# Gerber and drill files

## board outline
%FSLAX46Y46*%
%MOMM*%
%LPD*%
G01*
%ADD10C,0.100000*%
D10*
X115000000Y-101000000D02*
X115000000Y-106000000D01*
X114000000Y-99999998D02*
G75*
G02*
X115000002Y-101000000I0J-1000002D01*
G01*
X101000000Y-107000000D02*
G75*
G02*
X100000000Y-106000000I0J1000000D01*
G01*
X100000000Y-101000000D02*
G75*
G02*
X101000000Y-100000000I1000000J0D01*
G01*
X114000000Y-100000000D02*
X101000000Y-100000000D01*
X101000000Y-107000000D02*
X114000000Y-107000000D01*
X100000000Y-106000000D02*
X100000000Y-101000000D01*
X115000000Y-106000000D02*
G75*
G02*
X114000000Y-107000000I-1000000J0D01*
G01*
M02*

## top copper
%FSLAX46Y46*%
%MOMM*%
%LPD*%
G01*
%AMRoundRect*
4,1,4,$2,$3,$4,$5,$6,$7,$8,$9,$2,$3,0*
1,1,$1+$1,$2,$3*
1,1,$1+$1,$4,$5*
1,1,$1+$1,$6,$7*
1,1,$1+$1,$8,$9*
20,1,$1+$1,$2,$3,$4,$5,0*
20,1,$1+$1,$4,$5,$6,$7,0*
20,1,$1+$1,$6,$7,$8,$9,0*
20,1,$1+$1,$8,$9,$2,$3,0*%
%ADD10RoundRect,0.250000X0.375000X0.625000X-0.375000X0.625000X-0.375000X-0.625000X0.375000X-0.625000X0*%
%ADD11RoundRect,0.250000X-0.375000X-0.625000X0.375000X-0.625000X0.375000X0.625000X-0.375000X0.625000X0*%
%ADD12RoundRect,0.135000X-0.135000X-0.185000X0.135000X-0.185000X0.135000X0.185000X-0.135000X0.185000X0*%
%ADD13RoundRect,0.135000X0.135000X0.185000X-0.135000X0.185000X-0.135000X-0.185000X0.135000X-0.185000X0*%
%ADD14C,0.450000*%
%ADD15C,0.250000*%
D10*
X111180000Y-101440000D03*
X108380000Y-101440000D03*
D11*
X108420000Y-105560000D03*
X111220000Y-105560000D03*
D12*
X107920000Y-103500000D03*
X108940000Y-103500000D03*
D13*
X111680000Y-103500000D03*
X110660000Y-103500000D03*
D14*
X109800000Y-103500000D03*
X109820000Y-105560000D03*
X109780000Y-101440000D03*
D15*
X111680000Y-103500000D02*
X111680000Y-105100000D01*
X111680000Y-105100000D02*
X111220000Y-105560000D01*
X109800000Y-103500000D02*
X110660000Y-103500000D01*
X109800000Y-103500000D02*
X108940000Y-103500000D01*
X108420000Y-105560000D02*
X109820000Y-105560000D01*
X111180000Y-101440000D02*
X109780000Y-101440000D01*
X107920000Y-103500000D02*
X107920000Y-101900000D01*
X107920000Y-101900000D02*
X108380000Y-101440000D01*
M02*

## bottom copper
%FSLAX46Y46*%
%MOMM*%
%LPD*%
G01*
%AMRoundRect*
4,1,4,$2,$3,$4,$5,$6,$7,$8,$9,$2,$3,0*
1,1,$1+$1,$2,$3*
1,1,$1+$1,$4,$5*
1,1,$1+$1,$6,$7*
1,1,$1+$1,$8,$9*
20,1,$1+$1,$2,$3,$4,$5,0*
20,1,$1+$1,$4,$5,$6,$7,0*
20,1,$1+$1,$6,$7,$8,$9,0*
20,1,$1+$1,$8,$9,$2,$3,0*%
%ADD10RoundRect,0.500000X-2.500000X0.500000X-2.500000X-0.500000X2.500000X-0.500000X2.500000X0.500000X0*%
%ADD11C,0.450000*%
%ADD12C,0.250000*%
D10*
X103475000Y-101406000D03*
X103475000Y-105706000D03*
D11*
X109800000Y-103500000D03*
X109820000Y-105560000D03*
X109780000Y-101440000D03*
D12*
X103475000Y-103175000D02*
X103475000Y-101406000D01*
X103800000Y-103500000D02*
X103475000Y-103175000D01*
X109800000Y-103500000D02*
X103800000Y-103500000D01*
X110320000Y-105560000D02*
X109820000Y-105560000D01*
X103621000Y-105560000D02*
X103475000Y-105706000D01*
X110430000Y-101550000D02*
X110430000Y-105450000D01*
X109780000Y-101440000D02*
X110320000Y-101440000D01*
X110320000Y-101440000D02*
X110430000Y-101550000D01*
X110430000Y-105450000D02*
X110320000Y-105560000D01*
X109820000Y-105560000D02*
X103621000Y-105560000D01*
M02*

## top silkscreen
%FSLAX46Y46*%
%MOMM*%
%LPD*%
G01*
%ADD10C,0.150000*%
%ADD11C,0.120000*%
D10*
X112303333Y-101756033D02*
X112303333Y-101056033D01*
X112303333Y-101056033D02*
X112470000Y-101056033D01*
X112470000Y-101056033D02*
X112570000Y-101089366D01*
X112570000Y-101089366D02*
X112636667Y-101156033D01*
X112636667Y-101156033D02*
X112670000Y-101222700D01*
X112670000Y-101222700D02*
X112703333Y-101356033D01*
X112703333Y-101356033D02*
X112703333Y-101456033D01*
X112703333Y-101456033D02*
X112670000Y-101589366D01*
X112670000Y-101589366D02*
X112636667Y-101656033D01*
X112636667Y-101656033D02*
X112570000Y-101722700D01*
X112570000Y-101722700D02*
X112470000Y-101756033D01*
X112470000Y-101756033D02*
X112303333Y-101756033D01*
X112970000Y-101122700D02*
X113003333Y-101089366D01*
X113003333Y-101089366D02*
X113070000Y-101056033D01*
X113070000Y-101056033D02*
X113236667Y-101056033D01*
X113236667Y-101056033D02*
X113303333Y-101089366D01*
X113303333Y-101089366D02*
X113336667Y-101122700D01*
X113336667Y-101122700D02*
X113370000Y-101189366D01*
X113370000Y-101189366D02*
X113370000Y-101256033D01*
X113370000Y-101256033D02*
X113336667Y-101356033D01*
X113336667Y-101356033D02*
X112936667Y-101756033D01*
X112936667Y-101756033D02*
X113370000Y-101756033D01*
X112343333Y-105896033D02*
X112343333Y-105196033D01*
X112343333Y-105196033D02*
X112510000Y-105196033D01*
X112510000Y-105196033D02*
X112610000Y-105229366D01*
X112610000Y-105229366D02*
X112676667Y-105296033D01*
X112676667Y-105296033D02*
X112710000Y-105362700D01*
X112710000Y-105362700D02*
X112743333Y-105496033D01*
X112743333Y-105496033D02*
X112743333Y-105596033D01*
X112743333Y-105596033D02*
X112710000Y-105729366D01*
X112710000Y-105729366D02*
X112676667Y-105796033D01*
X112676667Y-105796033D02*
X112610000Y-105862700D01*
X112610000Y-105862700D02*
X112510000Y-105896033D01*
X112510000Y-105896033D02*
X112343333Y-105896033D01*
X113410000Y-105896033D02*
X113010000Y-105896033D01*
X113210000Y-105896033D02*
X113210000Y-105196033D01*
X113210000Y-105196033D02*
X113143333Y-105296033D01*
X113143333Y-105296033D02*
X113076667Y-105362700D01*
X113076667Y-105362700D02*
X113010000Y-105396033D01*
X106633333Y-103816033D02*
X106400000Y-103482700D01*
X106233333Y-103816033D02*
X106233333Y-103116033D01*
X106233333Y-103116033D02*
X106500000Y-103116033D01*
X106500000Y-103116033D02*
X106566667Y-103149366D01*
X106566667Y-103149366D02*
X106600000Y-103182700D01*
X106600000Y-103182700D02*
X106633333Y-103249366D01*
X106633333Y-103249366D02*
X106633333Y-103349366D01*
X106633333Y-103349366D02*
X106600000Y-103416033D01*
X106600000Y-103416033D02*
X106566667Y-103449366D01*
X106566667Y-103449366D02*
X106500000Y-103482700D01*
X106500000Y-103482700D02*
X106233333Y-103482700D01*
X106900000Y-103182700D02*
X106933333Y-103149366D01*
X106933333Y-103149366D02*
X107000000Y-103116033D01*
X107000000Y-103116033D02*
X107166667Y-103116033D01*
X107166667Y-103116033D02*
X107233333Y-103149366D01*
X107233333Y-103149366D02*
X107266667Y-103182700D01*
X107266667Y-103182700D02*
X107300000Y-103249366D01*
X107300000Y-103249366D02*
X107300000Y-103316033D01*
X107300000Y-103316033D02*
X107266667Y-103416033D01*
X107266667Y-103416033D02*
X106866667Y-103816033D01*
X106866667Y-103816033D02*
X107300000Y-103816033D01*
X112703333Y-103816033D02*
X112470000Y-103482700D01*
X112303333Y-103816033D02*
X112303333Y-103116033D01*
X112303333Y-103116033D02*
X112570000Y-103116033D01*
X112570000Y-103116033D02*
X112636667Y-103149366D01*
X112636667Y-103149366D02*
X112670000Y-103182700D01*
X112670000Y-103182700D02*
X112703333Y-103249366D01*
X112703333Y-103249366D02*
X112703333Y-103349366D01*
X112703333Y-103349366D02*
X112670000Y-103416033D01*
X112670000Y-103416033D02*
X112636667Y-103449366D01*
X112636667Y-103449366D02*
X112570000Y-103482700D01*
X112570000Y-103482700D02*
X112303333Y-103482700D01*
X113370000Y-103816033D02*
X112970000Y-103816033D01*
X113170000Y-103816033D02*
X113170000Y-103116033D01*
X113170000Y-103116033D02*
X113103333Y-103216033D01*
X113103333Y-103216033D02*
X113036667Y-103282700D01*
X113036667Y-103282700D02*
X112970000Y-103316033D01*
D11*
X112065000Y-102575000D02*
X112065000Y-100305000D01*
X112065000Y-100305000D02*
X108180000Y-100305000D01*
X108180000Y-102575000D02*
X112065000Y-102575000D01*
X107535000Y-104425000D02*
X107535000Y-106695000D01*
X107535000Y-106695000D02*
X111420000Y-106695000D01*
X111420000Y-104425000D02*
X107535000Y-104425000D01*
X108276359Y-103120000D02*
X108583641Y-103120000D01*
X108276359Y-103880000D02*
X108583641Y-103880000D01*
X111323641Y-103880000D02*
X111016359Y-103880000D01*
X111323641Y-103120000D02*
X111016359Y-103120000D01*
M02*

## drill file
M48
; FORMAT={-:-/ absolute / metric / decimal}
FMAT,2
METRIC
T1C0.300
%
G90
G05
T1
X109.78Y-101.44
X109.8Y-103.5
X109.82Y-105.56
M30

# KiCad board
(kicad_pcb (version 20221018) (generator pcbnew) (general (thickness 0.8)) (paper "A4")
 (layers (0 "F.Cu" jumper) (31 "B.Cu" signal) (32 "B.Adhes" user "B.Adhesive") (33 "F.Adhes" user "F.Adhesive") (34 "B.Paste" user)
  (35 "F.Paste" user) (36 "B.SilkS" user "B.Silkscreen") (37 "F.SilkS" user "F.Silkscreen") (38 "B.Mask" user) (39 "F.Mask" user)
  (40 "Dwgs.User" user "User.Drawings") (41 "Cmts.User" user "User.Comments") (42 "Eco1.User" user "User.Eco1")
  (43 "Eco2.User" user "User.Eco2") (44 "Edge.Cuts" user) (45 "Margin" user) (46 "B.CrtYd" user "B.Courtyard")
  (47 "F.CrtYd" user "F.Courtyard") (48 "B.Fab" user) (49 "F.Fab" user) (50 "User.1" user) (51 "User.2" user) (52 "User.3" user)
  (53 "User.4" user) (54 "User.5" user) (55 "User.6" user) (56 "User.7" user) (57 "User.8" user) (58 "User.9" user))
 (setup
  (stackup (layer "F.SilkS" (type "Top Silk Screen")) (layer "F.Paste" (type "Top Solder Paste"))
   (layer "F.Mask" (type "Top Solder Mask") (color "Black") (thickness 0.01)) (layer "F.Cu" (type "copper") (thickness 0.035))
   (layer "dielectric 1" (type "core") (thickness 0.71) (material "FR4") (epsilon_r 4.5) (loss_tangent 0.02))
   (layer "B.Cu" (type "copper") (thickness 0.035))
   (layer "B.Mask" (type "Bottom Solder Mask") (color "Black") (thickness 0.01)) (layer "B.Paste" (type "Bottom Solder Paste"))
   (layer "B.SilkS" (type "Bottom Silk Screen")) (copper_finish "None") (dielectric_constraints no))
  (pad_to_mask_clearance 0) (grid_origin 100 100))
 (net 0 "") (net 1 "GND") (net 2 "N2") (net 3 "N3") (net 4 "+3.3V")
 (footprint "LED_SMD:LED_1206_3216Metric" (layer "F.Cu") (at 109.78 101.44 180)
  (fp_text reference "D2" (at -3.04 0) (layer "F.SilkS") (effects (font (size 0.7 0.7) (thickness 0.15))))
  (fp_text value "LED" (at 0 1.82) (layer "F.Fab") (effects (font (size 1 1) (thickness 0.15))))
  (fp_line (start -2.285 -1.135) (end -2.285 1.135) (stroke (width 0.12) (type solid)) (layer "F.SilkS"))
  (fp_line (start -2.285 1.135) (end 1.6 1.135) (stroke (width 0.12) (type solid)) (layer "F.SilkS"))
  (fp_line (start 1.6 -1.135) (end -2.285 -1.135) (stroke (width 0.12) (type solid)) (layer "F.SilkS"))
  (pad "1" smd roundrect (at -1.4 0 180) (size 1.25 1.75) (layers "F.Cu" "F.Paste" "F.Mask") (roundrect_rratio 0.2) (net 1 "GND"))
  (pad "2" smd roundrect (at 1.4 0 180) (size 1.25 1.75) (layers "F.Cu" "F.Paste" "F.Mask") (roundrect_rratio 0.2) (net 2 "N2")))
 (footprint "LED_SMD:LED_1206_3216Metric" (layer "F.Cu") (at 109.82 105.56)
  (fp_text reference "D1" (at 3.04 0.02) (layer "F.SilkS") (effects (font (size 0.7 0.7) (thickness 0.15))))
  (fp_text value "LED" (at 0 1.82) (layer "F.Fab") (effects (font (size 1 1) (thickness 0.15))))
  (fp_line (start -2.285 -1.135) (end -2.285 1.135) (stroke (width 0.12) (type solid)) (layer "F.SilkS"))
  (fp_line (start -2.285 1.135) (end 1.6 1.135) (stroke (width 0.12) (type solid)) (layer "F.SilkS"))
  (fp_line (start 1.6 -1.135) (end -2.285 -1.135) (stroke (width 0.12) (type solid)) (layer "F.SilkS"))
  (pad "1" smd roundrect (at -1.4 0) (size 1.25 1.75) (layers "F.Cu" "F.Paste" "F.Mask") (roundrect_rratio 0.2) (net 1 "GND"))
  (pad "2" smd roundrect (at 1.4 0) (size 1.25 1.75) (layers "F.Cu" "F.Paste" "F.Mask") (roundrect_rratio 0.2) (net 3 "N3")))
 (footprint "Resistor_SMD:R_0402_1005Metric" (layer "F.Cu") (at 108.43 103.5)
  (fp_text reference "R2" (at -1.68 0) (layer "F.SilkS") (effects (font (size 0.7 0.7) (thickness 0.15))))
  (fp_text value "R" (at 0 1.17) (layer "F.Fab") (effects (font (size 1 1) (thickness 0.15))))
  (fp_line (start -0.153641 -0.38) (end 0.153641 -0.38) (stroke (width 0.12) (type solid)) (layer "F.SilkS"))
  (fp_line (start -0.153641 0.38) (end 0.153641 0.38) (stroke (width 0.12) (type solid)) (layer "F.SilkS"))
  (pad "1" smd roundrect (at -0.51 0) (size 0.54 0.64) (layers "F.Cu" "F.Paste" "F.Mask") (roundrect_rratio 0.25) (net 2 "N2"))
  (pad "2" smd roundrect (at 0.51 0) (size 0.54 0.64) (layers "F.Cu" "F.Paste" "F.Mask") (roundrect_rratio 0.25) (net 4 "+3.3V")))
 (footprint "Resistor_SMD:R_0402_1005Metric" (layer "F.Cu") (at 111.17 103.5 180)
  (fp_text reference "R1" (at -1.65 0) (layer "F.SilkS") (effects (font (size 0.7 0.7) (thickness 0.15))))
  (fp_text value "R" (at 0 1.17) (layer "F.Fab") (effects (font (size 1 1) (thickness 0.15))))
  (fp_line (start -0.153641 -0.38) (end 0.153641 -0.38) (stroke (width 0.12) (type solid)) (layer "F.SilkS"))
  (fp_line (start -0.153641 0.38) (end 0.153641 0.38) (stroke (width 0.12) (type solid)) (layer "F.SilkS"))
  (pad "1" smd roundrect (at -0.51 0 180) (size 0.54 0.64) (layers "F.Cu" "F.Paste" "F.Mask") (roundrect_rratio 0.25) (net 3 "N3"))
  (pad "2" smd roundrect (at 0.51 0 180) (size 0.54 0.64) (layers "F.Cu" "F.Paste" "F.Mask") (roundrect_rratio 0.25) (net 4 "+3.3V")))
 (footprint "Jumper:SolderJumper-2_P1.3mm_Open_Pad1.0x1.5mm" (layer "B.Cu") (at 103.475 103.556 -90)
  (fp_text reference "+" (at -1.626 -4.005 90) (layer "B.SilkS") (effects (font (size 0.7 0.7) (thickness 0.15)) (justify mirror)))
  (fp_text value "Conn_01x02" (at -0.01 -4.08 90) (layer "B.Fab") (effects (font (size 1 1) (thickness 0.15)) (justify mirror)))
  (pad "1" smd roundrect (at -2.15 0 270) (size 2 6) (layers "B.Cu" "B.Mask") (roundrect_rratio 0.25) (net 4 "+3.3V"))
  (pad "2" smd roundrect (at 2.15 0 270) (size 2 6) (layers "B.Cu" "B.Mask") (roundrect_rratio 0.25) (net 1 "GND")))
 (gr_line (start 115 101) (end 115 106) (stroke (width 0.1) (type default)) (layer "Edge.Cuts"))
 (gr_arc (start 114 99.999998) (mid 114.707107 100.292892) (end 115 101) (stroke (width 0.1) (type default)) (layer "Edge.Cuts"))
 (gr_arc (start 101 107) (mid 100.292894 106.707107) (end 100 106) (stroke (width 0.1) (type default)) (layer "Edge.Cuts"))
 (gr_arc (start 100 101) (mid 100.292893 100.292894) (end 101 100.000002) (stroke (width 0.1) (type default)) (layer "Edge.Cuts"))
 (gr_line (start 114 100) (end 101 100) (stroke (width 0.1) (type default)) (layer "Edge.Cuts"))
 (gr_line (start 101 107) (end 114 107) (stroke (width 0.1) (type default)) (layer "Edge.Cuts"))
 (gr_line (start 100 106) (end 100 101) (stroke (width 0.1) (type default)) (layer "Edge.Cuts"))
 (gr_arc (start 115 106) (mid 114.707106 106.707106) (end 114 107) (stroke (width 0.1) (type default)) (layer "Edge.Cuts"))
 (segment (start 111.68 103.5) (end 111.68 105.1) (width 0.25) (layer "F.Cu") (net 3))
 (segment (start 111.68 105.1) (end 111.22 105.56) (width 0.25) (layer "F.Cu") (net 3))
 (segment (start 109.8 103.5) (end 110.66 103.5) (width 0.25) (layer "F.Cu") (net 4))
 (segment (start 109.8 103.5) (end 108.94 103.5) (width 0.25) (layer "F.Cu") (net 4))
 (via (at 109.8 103.5) (size 0.45) (drill 0.3) (layers "F.Cu" "B.Cu") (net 4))
 (segment (start 103.475 103.175) (end 103.475 101.406) (width 0.25) (layer "B.Cu") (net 4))
 (segment (start 103.8 103.5) (end 103.475 103.175) (width 0.25) (layer "B.Cu") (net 4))
 (segment (start 109.8 103.5) (end 103.8 103.5) (width 0.25) (layer "B.Cu") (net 4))
 (segment (start 108.42 105.56) (end 109.82 105.56) (width 0.25) (layer "F.Cu") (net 1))
 (segment (start 111.18 101.44) (end 109.78 101.44) (width 0.25) (layer "F.Cu") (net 1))
 (via (at 109.82 105.56) (size 0.45) (drill 0.3) (layers "F.Cu" "B.Cu") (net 1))
 (via (at 109.78 101.44) (size 0.45) (drill 0.3) (layers "F.Cu" "B.Cu") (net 1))
 (segment (start 110.32 105.56) (end 109.82 105.56) (width 0.25) (layer "B.Cu") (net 1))
 (segment (start 103.621 105.56) (end 103.475 105.706) (width 0.25) (layer "B.Cu") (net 1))
 (segment (start 110.43 101.55) (end 110.43 105.45) (width 0.25) (layer "B.Cu") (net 1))
 (segment (start 109.78 101.44) (end 110.32 101.44) (width 0.25) (layer "B.Cu") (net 1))
 (segment (start 110.32 101.44) (end 110.43 101.55) (width 0.25) (layer "B.Cu") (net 1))
 (segment (start 110.43 105.45) (end 110.32 105.56) (width 0.25) (layer "B.Cu") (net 1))
 (segment (start 109.82 105.56) (end 103.621 105.56) (width 0.25) (layer "B.Cu") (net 1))
 (segment (start 107.92 103.5) (end 107.92 101.9) (width 0.25) (layer "F.Cu") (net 2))
 (segment (start 107.92 101.9) (end 108.38 101.44) (width 0.25) (layer "F.Cu") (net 2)))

